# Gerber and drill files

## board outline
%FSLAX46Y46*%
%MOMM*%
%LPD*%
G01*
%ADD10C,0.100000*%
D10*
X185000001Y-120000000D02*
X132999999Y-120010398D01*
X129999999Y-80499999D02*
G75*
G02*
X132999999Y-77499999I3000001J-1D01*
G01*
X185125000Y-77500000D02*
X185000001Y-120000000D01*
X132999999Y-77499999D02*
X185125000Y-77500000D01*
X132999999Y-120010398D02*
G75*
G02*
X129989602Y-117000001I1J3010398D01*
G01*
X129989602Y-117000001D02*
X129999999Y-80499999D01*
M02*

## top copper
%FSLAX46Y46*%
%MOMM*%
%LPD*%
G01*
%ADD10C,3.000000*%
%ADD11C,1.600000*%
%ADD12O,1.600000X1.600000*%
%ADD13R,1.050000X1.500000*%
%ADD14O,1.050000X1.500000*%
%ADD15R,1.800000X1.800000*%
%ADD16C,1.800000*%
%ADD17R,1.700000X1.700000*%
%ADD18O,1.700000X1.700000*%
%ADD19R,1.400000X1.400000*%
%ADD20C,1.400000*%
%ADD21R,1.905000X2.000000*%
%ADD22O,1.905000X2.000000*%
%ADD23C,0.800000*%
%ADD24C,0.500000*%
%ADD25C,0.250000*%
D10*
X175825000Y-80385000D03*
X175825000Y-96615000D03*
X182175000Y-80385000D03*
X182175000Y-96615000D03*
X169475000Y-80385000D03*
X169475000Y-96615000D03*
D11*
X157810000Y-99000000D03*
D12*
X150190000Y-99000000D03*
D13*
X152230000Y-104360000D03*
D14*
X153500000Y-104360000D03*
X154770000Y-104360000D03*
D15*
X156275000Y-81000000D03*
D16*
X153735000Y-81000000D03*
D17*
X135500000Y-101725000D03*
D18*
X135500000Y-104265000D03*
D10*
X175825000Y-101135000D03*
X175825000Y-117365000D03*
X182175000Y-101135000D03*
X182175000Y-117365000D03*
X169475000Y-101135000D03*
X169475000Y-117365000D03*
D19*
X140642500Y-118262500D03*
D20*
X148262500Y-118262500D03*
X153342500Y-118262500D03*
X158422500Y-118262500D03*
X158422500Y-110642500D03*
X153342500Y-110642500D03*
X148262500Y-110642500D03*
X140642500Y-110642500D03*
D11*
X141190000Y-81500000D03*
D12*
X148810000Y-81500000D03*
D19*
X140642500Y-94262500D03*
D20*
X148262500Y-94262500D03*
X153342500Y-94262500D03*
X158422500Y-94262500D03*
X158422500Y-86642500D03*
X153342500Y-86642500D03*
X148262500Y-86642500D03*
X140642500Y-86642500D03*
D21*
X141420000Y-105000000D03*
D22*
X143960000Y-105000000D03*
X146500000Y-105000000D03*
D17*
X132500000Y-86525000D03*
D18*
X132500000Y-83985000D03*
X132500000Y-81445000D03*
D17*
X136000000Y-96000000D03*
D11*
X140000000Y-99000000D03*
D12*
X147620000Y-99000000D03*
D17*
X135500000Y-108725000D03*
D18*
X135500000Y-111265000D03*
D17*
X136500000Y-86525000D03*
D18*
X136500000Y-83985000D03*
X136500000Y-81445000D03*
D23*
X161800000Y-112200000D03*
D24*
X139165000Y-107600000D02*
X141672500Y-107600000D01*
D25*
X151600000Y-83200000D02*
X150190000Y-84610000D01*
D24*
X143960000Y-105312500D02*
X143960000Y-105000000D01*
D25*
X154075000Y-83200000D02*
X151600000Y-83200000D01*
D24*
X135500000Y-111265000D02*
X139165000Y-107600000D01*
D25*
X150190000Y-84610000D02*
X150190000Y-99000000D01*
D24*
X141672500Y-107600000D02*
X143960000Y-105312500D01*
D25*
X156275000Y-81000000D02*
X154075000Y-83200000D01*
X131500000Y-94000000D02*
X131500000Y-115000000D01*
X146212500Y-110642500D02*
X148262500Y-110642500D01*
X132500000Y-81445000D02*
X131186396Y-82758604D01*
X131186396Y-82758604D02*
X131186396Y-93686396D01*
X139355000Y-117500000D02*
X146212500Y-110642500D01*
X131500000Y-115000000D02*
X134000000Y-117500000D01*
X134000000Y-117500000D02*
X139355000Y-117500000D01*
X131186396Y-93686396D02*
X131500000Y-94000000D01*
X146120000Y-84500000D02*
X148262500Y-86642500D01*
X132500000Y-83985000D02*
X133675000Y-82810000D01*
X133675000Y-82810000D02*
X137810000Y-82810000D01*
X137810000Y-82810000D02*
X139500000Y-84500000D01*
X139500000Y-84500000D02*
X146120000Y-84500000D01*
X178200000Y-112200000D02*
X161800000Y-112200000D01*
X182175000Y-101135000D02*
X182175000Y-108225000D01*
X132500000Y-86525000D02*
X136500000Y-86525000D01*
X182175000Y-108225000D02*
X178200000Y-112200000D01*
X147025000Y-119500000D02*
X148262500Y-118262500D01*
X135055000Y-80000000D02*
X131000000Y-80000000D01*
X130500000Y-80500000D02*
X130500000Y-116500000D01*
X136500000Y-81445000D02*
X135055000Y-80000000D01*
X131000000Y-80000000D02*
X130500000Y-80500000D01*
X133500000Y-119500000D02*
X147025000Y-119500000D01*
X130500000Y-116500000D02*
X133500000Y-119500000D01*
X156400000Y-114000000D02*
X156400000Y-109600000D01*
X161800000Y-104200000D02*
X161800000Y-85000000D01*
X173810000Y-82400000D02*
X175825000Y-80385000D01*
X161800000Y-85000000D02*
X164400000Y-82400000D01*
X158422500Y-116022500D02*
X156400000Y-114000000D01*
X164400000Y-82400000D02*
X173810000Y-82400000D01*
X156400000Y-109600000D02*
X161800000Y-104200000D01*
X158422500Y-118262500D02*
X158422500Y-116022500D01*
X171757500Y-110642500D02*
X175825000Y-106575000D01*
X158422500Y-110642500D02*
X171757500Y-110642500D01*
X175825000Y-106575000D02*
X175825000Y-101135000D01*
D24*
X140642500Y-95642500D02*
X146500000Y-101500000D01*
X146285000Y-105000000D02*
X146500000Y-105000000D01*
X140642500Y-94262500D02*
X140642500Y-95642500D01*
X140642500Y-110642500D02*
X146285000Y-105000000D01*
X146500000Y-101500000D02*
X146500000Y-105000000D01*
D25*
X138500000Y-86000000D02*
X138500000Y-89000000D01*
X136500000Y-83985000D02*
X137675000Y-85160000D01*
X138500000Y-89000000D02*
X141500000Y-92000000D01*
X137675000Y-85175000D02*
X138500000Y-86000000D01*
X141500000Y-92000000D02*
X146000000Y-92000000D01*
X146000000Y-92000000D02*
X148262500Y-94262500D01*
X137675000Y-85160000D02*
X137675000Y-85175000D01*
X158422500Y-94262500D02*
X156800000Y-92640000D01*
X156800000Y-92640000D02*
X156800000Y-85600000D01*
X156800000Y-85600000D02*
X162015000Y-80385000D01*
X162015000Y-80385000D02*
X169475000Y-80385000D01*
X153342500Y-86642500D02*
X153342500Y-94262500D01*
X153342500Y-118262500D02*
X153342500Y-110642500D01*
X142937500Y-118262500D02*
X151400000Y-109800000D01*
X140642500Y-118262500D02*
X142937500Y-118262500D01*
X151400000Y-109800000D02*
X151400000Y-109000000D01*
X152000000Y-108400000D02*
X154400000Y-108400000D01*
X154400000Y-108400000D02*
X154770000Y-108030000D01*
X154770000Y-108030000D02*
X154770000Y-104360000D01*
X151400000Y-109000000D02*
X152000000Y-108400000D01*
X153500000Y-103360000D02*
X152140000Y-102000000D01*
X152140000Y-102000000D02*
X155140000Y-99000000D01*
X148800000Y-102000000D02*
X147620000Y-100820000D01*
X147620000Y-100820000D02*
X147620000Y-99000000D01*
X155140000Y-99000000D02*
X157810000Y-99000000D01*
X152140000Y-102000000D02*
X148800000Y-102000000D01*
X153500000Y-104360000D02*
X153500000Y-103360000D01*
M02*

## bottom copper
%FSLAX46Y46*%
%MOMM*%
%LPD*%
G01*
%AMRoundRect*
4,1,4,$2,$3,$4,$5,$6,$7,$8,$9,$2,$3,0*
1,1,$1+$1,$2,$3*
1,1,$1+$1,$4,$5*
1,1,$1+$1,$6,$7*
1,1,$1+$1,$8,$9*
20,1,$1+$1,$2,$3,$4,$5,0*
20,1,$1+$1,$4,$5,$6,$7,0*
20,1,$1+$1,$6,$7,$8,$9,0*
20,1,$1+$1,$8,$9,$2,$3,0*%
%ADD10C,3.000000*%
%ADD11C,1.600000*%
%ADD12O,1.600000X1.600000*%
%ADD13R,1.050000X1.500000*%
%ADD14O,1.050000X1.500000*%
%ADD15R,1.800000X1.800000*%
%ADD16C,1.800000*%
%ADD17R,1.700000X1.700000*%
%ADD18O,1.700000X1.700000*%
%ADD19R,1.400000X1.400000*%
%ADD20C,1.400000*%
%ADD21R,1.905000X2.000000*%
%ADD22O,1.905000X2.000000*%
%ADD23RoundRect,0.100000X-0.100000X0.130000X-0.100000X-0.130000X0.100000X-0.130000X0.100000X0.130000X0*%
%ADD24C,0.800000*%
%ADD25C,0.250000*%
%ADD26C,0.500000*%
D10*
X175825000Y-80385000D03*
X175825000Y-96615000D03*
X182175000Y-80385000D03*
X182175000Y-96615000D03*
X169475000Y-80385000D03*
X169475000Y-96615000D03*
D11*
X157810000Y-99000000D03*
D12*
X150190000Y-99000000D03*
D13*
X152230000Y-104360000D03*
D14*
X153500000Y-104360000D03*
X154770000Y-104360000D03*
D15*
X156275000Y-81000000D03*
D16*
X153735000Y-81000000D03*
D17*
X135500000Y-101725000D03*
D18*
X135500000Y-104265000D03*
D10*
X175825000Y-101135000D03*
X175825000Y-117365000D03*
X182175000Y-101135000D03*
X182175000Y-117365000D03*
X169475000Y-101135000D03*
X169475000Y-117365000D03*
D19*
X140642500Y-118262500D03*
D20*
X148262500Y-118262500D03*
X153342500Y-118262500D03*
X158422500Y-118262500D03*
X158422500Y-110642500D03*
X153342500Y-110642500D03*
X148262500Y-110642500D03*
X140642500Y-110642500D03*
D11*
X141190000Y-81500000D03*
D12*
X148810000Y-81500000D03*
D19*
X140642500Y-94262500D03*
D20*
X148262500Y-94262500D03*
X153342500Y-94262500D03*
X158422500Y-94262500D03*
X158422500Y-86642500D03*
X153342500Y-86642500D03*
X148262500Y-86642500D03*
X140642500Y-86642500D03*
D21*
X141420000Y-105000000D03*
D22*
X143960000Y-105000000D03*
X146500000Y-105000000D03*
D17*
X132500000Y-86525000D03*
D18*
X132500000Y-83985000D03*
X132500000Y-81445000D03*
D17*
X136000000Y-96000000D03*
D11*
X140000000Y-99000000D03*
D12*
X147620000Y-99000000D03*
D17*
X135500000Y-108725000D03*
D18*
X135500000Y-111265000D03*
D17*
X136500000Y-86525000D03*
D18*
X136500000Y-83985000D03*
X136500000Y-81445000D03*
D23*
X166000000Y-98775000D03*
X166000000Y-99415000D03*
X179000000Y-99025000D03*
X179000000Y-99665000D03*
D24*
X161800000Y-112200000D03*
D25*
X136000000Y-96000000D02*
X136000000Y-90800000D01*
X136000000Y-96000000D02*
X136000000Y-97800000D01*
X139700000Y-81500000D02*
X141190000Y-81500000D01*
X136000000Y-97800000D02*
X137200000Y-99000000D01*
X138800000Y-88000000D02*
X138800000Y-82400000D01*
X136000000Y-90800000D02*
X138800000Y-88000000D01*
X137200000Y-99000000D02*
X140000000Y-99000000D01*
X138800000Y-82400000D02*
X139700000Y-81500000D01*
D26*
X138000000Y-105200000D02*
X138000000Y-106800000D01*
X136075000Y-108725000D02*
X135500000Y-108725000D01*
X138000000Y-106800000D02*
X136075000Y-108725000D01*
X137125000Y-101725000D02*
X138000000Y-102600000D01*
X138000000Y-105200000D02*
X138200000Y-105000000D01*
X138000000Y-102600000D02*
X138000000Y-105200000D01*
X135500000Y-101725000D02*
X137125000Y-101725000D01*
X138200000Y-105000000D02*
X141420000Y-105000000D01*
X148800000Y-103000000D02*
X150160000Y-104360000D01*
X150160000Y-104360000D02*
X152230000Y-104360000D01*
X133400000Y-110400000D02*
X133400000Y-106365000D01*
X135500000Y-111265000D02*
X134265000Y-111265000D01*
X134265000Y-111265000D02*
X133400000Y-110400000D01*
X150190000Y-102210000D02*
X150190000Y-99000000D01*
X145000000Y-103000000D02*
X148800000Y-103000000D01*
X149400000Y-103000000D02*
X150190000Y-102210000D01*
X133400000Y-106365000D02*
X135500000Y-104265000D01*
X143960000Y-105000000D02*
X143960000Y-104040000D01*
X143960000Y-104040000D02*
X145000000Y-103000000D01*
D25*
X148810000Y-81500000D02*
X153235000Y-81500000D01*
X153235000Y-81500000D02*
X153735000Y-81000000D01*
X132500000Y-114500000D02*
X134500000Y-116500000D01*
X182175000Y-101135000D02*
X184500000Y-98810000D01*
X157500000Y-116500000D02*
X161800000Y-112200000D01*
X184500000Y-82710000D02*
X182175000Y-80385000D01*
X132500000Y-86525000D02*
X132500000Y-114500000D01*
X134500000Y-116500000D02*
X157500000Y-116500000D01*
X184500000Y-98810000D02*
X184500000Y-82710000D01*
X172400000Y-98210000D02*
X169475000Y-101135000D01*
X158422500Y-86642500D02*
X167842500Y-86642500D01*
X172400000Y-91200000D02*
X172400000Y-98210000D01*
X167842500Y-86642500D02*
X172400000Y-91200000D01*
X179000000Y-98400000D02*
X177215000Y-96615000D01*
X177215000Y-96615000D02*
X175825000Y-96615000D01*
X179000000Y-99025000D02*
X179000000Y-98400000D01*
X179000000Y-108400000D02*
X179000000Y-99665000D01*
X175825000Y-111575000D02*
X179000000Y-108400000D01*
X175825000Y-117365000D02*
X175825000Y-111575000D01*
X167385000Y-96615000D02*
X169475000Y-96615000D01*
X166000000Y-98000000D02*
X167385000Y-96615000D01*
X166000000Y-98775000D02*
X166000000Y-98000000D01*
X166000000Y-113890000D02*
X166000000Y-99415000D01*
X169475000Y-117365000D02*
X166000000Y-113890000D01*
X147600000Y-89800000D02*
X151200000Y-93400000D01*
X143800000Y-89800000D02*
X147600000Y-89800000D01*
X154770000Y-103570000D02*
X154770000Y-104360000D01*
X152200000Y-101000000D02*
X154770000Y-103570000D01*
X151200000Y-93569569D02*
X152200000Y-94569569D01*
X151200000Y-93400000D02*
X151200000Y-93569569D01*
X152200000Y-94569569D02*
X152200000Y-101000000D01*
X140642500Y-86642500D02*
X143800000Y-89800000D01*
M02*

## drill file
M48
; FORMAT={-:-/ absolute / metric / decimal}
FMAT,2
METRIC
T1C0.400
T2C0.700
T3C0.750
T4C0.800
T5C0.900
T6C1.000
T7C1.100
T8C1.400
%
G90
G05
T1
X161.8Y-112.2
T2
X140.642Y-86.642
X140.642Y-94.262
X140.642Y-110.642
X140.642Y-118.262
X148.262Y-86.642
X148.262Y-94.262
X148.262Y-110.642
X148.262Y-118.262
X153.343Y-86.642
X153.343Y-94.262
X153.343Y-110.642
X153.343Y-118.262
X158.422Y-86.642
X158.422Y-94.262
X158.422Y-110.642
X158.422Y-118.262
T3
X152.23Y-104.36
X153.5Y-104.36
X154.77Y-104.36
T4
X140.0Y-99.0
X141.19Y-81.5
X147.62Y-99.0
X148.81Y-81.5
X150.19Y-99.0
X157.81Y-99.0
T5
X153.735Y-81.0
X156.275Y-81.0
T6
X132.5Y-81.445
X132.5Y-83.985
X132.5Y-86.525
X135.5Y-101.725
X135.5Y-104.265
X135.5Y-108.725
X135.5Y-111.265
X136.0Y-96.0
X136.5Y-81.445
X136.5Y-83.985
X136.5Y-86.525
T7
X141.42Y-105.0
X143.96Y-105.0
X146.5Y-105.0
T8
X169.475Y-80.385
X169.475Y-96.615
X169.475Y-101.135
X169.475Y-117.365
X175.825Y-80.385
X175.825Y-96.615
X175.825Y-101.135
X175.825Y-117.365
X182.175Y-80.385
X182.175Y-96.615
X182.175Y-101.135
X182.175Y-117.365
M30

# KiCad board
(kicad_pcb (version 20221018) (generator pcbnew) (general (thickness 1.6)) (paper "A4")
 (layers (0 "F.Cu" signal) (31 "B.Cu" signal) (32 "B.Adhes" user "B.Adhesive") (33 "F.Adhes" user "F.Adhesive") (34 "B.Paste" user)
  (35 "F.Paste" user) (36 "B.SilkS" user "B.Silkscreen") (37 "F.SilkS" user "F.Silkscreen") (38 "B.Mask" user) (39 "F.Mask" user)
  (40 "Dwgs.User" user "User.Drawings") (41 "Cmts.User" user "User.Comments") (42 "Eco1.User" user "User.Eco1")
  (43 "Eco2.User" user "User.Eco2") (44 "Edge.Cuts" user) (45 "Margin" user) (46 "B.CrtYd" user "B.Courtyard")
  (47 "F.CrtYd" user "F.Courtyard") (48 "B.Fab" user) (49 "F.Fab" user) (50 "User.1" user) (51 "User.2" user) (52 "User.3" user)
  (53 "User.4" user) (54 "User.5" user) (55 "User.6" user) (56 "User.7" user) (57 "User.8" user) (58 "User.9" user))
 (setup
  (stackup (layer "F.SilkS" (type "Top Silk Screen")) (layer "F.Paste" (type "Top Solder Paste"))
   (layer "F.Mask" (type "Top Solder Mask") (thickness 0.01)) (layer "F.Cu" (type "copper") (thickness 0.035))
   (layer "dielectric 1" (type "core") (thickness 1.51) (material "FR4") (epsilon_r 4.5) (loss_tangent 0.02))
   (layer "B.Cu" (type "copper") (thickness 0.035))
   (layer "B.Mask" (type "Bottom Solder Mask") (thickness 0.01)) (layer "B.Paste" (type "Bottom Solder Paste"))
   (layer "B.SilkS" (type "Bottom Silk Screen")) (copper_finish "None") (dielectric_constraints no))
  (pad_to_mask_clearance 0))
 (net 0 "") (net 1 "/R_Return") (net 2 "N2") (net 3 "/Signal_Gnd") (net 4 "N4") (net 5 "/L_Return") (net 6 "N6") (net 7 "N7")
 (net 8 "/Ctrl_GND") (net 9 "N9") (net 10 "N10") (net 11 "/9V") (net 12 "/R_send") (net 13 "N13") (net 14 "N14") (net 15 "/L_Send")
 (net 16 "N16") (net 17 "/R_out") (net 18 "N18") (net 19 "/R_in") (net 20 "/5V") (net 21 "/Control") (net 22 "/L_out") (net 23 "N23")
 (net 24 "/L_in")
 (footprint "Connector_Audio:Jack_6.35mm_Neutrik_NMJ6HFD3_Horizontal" (layer "F.Cu") (at 169.475 80.385)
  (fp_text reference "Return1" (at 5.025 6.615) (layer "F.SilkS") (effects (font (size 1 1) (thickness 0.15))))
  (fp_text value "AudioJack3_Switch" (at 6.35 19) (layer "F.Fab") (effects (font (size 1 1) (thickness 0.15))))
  (pad "R" thru_hole circle (at 6.35 0) (size 3 3) (drill 1.4) (layers "*.Cu" "*.Mask") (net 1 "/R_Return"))
  (pad "RN" thru_hole circle (at 6.35 16.23) (size 3 3) (drill 1.4) (layers "*.Cu" "*.Mask") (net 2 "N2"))
  (pad "S" thru_hole circle (at 12.7 0) (size 3 3) (drill 1.4) (layers "*.Cu" "*.Mask") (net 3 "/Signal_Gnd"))
  (pad "SN" thru_hole circle (at 12.7 16.23) (size 3 3) (drill 1.4) (layers "*.Cu" "*.Mask") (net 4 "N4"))
  (pad "T" thru_hole circle (at 0 0) (size 3 3) (drill 1.4) (layers "*.Cu" "*.Mask") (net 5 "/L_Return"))
  (pad "TN" thru_hole circle (at 0 16.23) (size 3 3) (drill 1.4) (layers "*.Cu" "*.Mask") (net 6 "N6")))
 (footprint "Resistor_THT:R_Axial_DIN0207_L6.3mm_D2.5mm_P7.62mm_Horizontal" (layer "F.Cu") (at 157.81 99 180)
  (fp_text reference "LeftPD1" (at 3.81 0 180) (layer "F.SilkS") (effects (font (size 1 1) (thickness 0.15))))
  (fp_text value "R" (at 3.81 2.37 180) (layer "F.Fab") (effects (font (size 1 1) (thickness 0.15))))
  (pad "1" thru_hole circle (at 0 0 180) (size 1.6 1.6) (drill 0.8) (layers "*.Cu" "*.Mask") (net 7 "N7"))
  (pad "2" thru_hole oval (at 7.62 0 180) (size 1.6 1.6) (drill 0.8) (layers "*.Cu" "*.Mask") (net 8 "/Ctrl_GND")))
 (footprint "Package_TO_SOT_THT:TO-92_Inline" (layer "F.Cu") (at 152.23 104.36)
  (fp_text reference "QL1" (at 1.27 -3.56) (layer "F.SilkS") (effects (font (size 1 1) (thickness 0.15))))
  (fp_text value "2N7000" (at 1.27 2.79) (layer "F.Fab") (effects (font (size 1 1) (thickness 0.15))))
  (pad "1" thru_hole rect (at 0 0) (size 1.05 1.5) (drill 0.75) (layers "*.Cu" "*.Mask") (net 8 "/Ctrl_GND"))
  (pad "2" thru_hole oval (at 1.27 0) (size 1.05 1.5) (drill 0.75) (layers "*.Cu" "*.Mask") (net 7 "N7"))
  (pad "3" thru_hole oval (at 2.54 0) (size 1.05 1.5) (drill 0.75) (layers "*.Cu" "*.Mask") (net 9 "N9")))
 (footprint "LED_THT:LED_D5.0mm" (layer "F.Cu") (at 156.275 81 180)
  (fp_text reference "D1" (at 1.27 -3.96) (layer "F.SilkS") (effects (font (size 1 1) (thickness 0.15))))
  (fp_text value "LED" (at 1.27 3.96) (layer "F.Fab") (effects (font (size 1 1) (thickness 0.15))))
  (pad "1" thru_hole rect (at 0 0 180) (size 1.8 1.8) (drill 0.9) (layers "*.Cu" "*.Mask") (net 8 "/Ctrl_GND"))
  (pad "2" thru_hole circle (at 2.54 0 180) (size 1.8 1.8) (drill 0.9) (layers "*.Cu" "*.Mask") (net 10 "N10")))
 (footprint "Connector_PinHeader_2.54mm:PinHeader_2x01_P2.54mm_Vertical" (layer "F.Cu") (at 135.5 101.725 -90)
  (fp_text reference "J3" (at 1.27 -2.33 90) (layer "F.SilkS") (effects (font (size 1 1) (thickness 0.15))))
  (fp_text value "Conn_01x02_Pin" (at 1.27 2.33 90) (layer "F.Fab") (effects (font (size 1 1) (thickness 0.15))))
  (pad "1" thru_hole rect (at 0 0 270) (size 1.7 1.7) (drill 1) (layers "*.Cu" "*.Mask") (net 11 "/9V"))
  (pad "2" thru_hole oval (at 2.54 0 270) (size 1.7 1.7) (drill 1) (layers "*.Cu" "*.Mask") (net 8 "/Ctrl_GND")))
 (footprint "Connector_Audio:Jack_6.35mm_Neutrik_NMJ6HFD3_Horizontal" (layer "F.Cu") (at 169.475 101.135)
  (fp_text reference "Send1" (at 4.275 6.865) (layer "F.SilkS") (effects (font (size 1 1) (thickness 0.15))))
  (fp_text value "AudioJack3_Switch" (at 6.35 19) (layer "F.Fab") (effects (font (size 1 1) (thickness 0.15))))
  (pad "R" thru_hole circle (at 6.35 0) (size 3 3) (drill 1.4) (layers "*.Cu" "*.Mask") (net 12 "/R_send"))
  (pad "RN" thru_hole circle (at 6.35 16.23) (size 3 3) (drill 1.4) (layers "*.Cu" "*.Mask") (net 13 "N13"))
  (pad "S" thru_hole circle (at 12.7 0) (size 3 3) (drill 1.4) (layers "*.Cu" "*.Mask") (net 3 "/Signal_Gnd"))
  (pad "SN" thru_hole circle (at 12.7 16.23) (size 3 3) (drill 1.4) (layers "*.Cu" "*.Mask") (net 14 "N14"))
  (pad "T" thru_hole circle (at 0 0) (size 3 3) (drill 1.4) (layers "*.Cu" "*.Mask") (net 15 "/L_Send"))
  (pad "TN" thru_hole circle (at 0 16.23) (size 3 3) (drill 1.4) (layers "*.Cu" "*.Mask") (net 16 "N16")))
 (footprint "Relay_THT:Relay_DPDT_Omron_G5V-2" (layer "F.Cu") (at 140.6425 118.2625 90)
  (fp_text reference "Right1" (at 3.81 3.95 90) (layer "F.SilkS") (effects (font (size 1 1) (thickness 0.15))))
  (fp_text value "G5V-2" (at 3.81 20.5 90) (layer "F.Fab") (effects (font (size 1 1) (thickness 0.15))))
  (pad "1" thru_hole rect (at 0 0 90) (size 1.4 1.4) (drill 0.7) (layers "*.Cu" "*.Mask") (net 9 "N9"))
  (pad "4" thru_hole circle (at 0 7.62 90) (size 1.4 1.4) (drill 0.7) (layers "*.Cu" "*.Mask") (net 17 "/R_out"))
  (pad "6" thru_hole circle (at 0 12.7 90) (size 1.4 1.4) (drill 0.7) (layers "*.Cu" "*.Mask") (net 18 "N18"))
  (pad "8" thru_hole circle (at 0 17.78 90) (size 1.4 1.4) (drill 0.7) (layers "*.Cu" "*.Mask") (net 1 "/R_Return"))
  (pad "9" thru_hole circle (at 7.62 17.78 90) (size 1.4 1.4) (drill 0.7) (layers "*.Cu" "*.Mask") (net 12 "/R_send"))
  (pad "11" thru_hole circle (at 7.62 12.7 90) (size 1.4 1.4) (drill 0.7) (layers "*.Cu" "*.Mask") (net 18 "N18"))
  (pad "13" thru_hole circle (at 7.62 7.62 90) (size 1.4 1.4) (drill 0.7) (layers "*.Cu" "*.Mask") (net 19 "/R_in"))
  (pad "16" thru_hole circle (at 7.62 0 90) (size 1.4 1.4) (drill 0.7) (layers "*.Cu" "*.Mask") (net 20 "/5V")))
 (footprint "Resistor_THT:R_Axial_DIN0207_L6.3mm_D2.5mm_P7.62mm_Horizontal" (layer "F.Cu") (at 141.19 81.5)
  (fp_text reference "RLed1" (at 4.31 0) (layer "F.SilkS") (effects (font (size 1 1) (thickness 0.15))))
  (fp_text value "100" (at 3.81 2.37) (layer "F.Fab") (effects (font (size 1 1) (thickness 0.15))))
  (pad "1" thru_hole circle (at 0 0) (size 1.6 1.6) (drill 0.8) (layers "*.Cu" "*.Mask") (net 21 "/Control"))
  (pad "2" thru_hole oval (at 7.62 0) (size 1.6 1.6) (drill 0.8) (layers "*.Cu" "*.Mask") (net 10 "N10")))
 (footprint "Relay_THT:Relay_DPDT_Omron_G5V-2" (layer "F.Cu") (at 140.6425 94.2625 90)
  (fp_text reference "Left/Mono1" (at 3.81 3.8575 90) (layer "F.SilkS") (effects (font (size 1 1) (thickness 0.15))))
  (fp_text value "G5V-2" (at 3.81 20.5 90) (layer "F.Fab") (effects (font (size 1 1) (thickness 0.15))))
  (pad "1" thru_hole rect (at 0 0 90) (size 1.4 1.4) (drill 0.7) (layers "*.Cu" "*.Mask") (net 20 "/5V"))
  (pad "4" thru_hole circle (at 0 7.62 90) (size 1.4 1.4) (drill 0.7) (layers "*.Cu" "*.Mask") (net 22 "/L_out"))
  (pad "6" thru_hole circle (at 0 12.7 90) (size 1.4 1.4) (drill 0.7) (layers "*.Cu" "*.Mask") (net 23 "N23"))
  (pad "8" thru_hole circle (at 0 17.78 90) (size 1.4 1.4) (drill 0.7) (layers "*.Cu" "*.Mask") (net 5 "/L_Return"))
  (pad "9" thru_hole circle (at 7.62 17.78 90) (size 1.4 1.4) (drill 0.7) (layers "*.Cu" "*.Mask") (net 15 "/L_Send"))
  (pad "11" thru_hole circle (at 7.62 12.7 90) (size 1.4 1.4) (drill 0.7) (layers "*.Cu" "*.Mask") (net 23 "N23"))
  (pad "13" thru_hole circle (at 7.62 7.62 90) (size 1.4 1.4) (drill 0.7) (layers "*.Cu" "*.Mask") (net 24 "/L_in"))
  (pad "16" thru_hole circle (at 7.62 0 90) (size 1.4 1.4) (drill 0.7) (layers "*.Cu" "*.Mask") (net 9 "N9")))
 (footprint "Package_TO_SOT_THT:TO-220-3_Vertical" (layer "F.Cu") (at 141.42 105)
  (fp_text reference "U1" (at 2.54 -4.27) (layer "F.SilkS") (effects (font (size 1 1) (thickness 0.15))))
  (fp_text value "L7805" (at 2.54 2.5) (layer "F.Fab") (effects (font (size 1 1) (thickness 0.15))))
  (pad "1" thru_hole rect (at 0 0) (size 1.905 2) (drill 1.1) (layers "*.Cu" "*.Mask") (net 11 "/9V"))
  (pad "2" thru_hole oval (at 2.54 0) (size 1.905 2) (drill 1.1) (layers "*.Cu" "*.Mask") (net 8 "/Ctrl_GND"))
  (pad "3" thru_hole oval (at 5.08 0) (size 1.905 2) (drill 1.1) (layers "*.Cu" "*.Mask") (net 20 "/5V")))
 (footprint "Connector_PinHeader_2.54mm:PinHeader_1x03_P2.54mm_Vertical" (layer "F.Cu") (at 132.5 86.525 180)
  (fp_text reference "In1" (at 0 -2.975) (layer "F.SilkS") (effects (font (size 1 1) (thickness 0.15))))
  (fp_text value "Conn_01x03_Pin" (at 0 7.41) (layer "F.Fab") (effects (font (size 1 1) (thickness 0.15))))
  (pad "1" thru_hole rect (at 0 0 180) (size 1.7 1.7) (drill 1) (layers "*.Cu" "*.Mask") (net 3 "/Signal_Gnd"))
  (pad "2" thru_hole oval (at 0 2.54 180) (size 1.7 1.7) (drill 1) (layers "*.Cu" "*.Mask") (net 24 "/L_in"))
  (pad "3" thru_hole oval (at 0 5.08 180) (size 1.7 1.7) (drill 1) (layers "*.Cu" "*.Mask") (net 19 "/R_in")))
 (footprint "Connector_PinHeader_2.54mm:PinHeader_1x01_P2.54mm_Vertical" (layer "F.Cu") (at 136 96)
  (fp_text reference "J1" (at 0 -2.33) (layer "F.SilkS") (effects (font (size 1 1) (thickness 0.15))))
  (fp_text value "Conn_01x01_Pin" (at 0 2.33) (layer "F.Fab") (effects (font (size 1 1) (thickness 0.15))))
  (pad "1" thru_hole rect (at 0 0) (size 1.7 1.7) (drill 1) (layers "*.Cu" "*.Mask") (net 21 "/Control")))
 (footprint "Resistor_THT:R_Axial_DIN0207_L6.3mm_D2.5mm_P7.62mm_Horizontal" (layer "F.Cu") (at 140 99)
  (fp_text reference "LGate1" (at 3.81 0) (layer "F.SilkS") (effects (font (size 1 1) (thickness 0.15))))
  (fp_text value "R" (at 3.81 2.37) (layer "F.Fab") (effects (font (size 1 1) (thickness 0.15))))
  (pad "1" thru_hole circle (at 0 0) (size 1.6 1.6) (drill 0.8) (layers "*.Cu" "*.Mask") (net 21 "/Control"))
  (pad "2" thru_hole oval (at 7.62 0) (size 1.6 1.6) (drill 0.8) (layers "*.Cu" "*.Mask") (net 7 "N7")))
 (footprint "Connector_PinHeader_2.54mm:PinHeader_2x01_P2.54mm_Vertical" (layer "F.Cu") (at 135.5 108.725 -90)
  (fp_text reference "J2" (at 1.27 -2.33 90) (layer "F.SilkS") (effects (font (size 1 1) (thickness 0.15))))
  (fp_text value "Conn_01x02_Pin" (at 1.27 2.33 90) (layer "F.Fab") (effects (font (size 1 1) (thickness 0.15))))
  (pad "1" thru_hole rect (at 0 0 270) (size 1.7 1.7) (drill 1) (layers "*.Cu" "*.Mask") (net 11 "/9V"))
  (pad "2" thru_hole oval (at 2.54 0 270) (size 1.7 1.7) (drill 1) (layers "*.Cu" "*.Mask") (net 8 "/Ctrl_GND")))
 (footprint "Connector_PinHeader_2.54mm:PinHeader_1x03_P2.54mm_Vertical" (layer "F.Cu") (at 136.5 86.525 180)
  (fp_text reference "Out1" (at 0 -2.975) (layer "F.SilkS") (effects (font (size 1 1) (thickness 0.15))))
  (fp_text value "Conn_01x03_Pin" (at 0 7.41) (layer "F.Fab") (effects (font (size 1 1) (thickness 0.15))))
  (pad "1" thru_hole rect (at 0 0 180) (size 1.7 1.7) (drill 1) (layers "*.Cu" "*.Mask") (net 3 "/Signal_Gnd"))
  (pad "2" thru_hole oval (at 0 2.54 180) (size 1.7 1.7) (drill 1) (layers "*.Cu" "*.Mask") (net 22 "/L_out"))
  (pad "3" thru_hole oval (at 0 5.08 180) (size 1.7 1.7) (drill 1) (layers "*.Cu" "*.Mask") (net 17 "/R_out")))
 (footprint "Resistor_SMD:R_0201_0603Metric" (layer "B.Cu") (at 166 99.095 -90)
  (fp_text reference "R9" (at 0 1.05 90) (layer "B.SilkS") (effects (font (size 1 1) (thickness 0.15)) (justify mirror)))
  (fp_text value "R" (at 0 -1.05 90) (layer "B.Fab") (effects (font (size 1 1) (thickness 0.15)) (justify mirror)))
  (pad "" smd roundrect (at -0.345 0 270) (size 0.318 0.36) (layers "B.Paste") (roundrect_rratio 0.25))
  (pad "" smd roundrect (at 0.345 0 270) (size 0.318 0.36) (layers "B.Paste") (roundrect_rratio 0.25))
  (pad "1" smd roundrect (at -0.32 0 270) (size 0.46 0.4) (layers "B.Cu" "B.Mask") (roundrect_rratio 0.25) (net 6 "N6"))
  (pad "2" smd roundrect (at 0.32 0 270) (size 0.46 0.4) (layers "B.Cu" "B.Mask") (roundrect_rratio 0.25) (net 16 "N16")))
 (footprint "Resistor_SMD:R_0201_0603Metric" (layer "B.Cu") (at 179 99.345 -90)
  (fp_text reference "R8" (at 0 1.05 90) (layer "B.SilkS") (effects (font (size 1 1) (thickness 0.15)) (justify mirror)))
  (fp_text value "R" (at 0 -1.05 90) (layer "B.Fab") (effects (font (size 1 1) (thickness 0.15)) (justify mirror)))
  (pad "" smd roundrect (at -0.345 0 270) (size 0.318 0.36) (layers "B.Paste") (roundrect_rratio 0.25))
  (pad "" smd roundrect (at 0.345 0 270) (size 0.318 0.36) (layers "B.Paste") (roundrect_rratio 0.25))
  (pad "1" smd roundrect (at -0.32 0 270) (size 0.46 0.4) (layers "B.Cu" "B.Mask") (roundrect_rratio 0.25) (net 2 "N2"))
  (pad "2" smd roundrect (at 0.32 0 270) (size 0.46 0.4) (layers "B.Cu" "B.Mask") (roundrect_rratio 0.25) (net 13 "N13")))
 (gr_line (start 185.000001 120) (end 132.999999 120.010398) (stroke (width 0.1) (type default)) (layer "Edge.Cuts"))
 (gr_arc (start 129.999999 80.499999) (mid 130.878679 78.378679) (end 132.999999 77.499999) (stroke (width 0.1) (type default))
  (layer "Edge.Cuts"))
 (gr_line (start 185.125 77.5) (end 185.000001 120) (stroke (width 0.1) (type default)) (layer "Edge.Cuts"))
 (gr_line (start 132.999999 77.499999) (end 185.125 77.5) (stroke (width 0.1) (type default)) (layer "Edge.Cuts"))
 (gr_arc (start 132.999999 120.010398) (mid 130.871327 119.128673) (end 129.989602 117.000001) (stroke (width 0.1) (type default))
  (layer "Edge.Cuts"))
 (gr_line (start 129.989602 117.000001) (end 129.999999 80.499999) (stroke (width 0.1) (type default)) (layer "Edge.Cuts"))
 (segment (start 136 96) (end 136 90.8) (width 0.25) (layer "B.Cu") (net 21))
 (segment (start 136 96) (end 136 97.8) (width 0.25) (layer "B.Cu") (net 21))
 (segment (start 139.7 81.5) (end 141.19 81.5) (width 0.25) (layer "B.Cu") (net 21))
 (segment (start 136 97.8) (end 137.2 99) (width 0.25) (layer "B.Cu") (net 21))
 (segment (start 138.8 88) (end 138.8 82.4) (width 0.25) (layer "B.Cu") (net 21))
 (segment (start 136 90.8) (end 138.8 88) (width 0.25) (layer "B.Cu") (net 21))
 (segment (start 137.2 99) (end 140 99) (width 0.25) (layer "B.Cu") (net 21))
 (segment (start 138.8 82.4) (end 139.7 81.5) (width 0.25) (layer "B.Cu") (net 21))
 (segment (start 138 105.2) (end 138 106.8) (width 0.5) (layer "B.Cu") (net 11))
 (segment (start 136.075 108.725) (end 135.5 108.725) (width 0.5) (layer "B.Cu") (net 11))
 (segment (start 138 106.8) (end 136.075 108.725) (width 0.5) (layer "B.Cu") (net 11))
 (segment (start 137.125 101.725) (end 138 102.6) (width 0.5) (layer "B.Cu") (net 11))
 (segment (start 138 105.2) (end 138.2 105) (width 0.5) (layer "B.Cu") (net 11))
 (segment (start 138 102.6) (end 138 105.2) (width 0.5) (layer "B.Cu") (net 11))
 (segment (start 135.5 101.725) (end 137.125 101.725) (width 0.5) (layer "B.Cu") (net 11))
 (segment (start 138.2 105) (end 141.42 105) (width 0.5) (layer "B.Cu") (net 11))
 (segment (start 139.165 107.6) (end 141.6725 107.6) (width 0.5) (layer "F.Cu") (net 8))
 (segment (start 151.6 83.2) (end 150.19 84.61) (width 0.25) (layer "F.Cu") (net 8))
 (segment (start 143.96 105.3125) (end 143.96 105) (width 0.5) (layer "F.Cu") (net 8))
 (segment (start 154.075 83.2) (end 151.6 83.2) (width 0.25) (layer "F.Cu") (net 8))
 (segment (start 135.5 111.265) (end 139.165 107.6) (width 0.5) (layer "F.Cu") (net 8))
 (segment (start 150.19 84.61) (end 150.19 99) (width 0.25) (layer "F.Cu") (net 8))
 (segment (start 141.6725 107.6) (end 143.96 105.3125) (width 0.5) (layer "F.Cu") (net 8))
 (segment (start 156.275 81) (end 154.075 83.2) (width 0.25) (layer "F.Cu") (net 8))
 (segment (start 148.8 103) (end 150.16 104.36) (width 0.5) (layer "B.Cu") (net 8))
 (segment (start 150.16 104.36) (end 152.23 104.36) (width 0.5) (layer "B.Cu") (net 8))
 (segment (start 133.4 110.4) (end 133.4 106.365) (width 0.5) (layer "B.Cu") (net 8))
 (segment (start 135.5 111.265) (end 134.265 111.265) (width 0.5) (layer "B.Cu") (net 8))
 (segment (start 134.265 111.265) (end 133.4 110.4) (width 0.5) (layer "B.Cu") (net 8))
 (segment (start 150.19 102.21) (end 150.19 99) (width 0.5) (layer "B.Cu") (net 8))
 (segment (start 145 103) (end 148.8 103) (width 0.5) (layer "B.Cu") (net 8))
 (segment (start 149.4 103) (end 150.19 102.21) (width 0.5) (layer "B.Cu") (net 8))
 (segment (start 133.4 106.365) (end 135.5 104.265) (width 0.5) (layer "B.Cu") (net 8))
 (segment (start 143.96 105) (end 143.96 104.04) (width 0.5) (layer "B.Cu") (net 8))
 (segment (start 143.96 104.04) (end 145 103) (width 0.5) (layer "B.Cu") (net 8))
 (segment (start 148.81 81.5) (end 153.235 81.5) (width 0.25) (layer "B.Cu") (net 10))
 (segment (start 153.235 81.5) (end 153.735 81) (width 0.25) (layer "B.Cu") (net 10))
 (segment (start 131.5 94) (end 131.5 115) (width 0.25) (layer "F.Cu") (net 19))
 (segment (start 146.2125 110.6425) (end 148.2625 110.6425) (width 0.25) (layer "F.Cu") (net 19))
 (segment (start 132.5 81.445) (end 131.186396 82.758604) (width 0.25) (layer "F.Cu") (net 19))
 (segment (start 131.186396 82.758604) (end 131.186396 93.686396) (width 0.25) (layer "F.Cu") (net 19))
 (segment (start 139.355 117.5) (end 146.2125 110.6425) (width 0.25) (layer "F.Cu") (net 19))
 (segment (start 131.5 115) (end 134 117.5) (width 0.25) (layer "F.Cu") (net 19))
 (segment (start 134 117.5) (end 139.355 117.5) (width 0.25) (layer "F.Cu") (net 19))
 (segment (start 131.186396 93.686396) (end 131.5 94) (width 0.25) (layer "F.Cu") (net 19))
 (segment (start 146.12 84.5) (end 148.2625 86.6425) (width 0.25) (layer "F.Cu") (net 24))
 (segment (start 132.5 83.985) (end 133.675 82.81) (width 0.25) (layer "F.Cu") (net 24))
 (segment (start 133.675 82.81) (end 137.81 82.81) (width 0.25) (layer "F.Cu") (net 24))
 (segment (start 137.81 82.81) (end 139.5 84.5) (width 0.25) (layer "F.Cu") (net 24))
 (segment (start 139.5 84.5) (end 146.12 84.5) (width 0.25) (layer "F.Cu") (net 24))
 (segment (start 178.2 112.2) (end 161.8 112.2) (width 0.25) (layer "F.Cu") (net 3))
 (segment (start 182.175 101.135) (end 182.175 108.225) (width 0.25) (layer "F.Cu") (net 3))
 (segment (start 132.5 86.525) (end 136.5 86.525) (width 0.25) (layer "F.Cu") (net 3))
 (segment (start 182.175 108.225) (end 178.2 112.2) (width 0.25) (layer "F.Cu") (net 3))
 (via (at 161.8 112.2) (size 0.8) (drill 0.4) (layers "F.Cu" "B.Cu") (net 3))
 (segment (start 132.5 114.5) (end 134.5 116.5) (width 0.25) (layer "B.Cu") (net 3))
 (segment (start 182.175 101.135) (end 184.5 98.81) (width 0.25) (layer "B.Cu") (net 3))
 (segment (start 157.5 116.5) (end 161.8 112.2) (width 0.25) (layer "B.Cu") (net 3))
 (segment (start 184.5 82.71) (end 182.175 80.385) (width 0.25) (layer "B.Cu") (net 3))
 (segment (start 132.5 86.525) (end 132.5 114.5) (width 0.25) (layer "B.Cu") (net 3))
 (segment (start 134.5 116.5) (end 157.5 116.5) (width 0.25) (layer "B.Cu") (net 3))
 (segment (start 184.5 98.81) (end 184.5 82.71) (width 0.25) (layer "B.Cu") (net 3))
 (segment (start 147.025 119.5) (end 148.2625 118.2625) (width 0.25) (layer "F.Cu") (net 17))
 (segment (start 135.055 80) (end 131 80) (width 0.25) (layer "F.Cu") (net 17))
 (segment (start 130.5 80.5) (end 130.5 116.5) (width 0.25) (layer "F.Cu") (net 17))
 (segment (start 136.5 81.445) (end 135.055 80) (width 0.25) (layer "F.Cu") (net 17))
 (segment (start 131 80) (end 130.5 80.5) (width 0.25) (layer "F.Cu") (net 17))
 (segment (start 133.5 119.5) (end 147.025 119.5) (width 0.25) (layer "F.Cu") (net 17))
 (segment (start 130.5 116.5) (end 133.5 119.5) (width 0.25) (layer "F.Cu") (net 17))
 (segment (start 156.4 114) (end 156.4 109.6) (width 0.25) (layer "F.Cu") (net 1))
 (segment (start 161.8 104.2) (end 161.8 85) (width 0.25) (layer "F.Cu") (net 1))
 (segment (start 173.81 82.4) (end 175.825 80.385) (width 0.25) (layer "F.Cu") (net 1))
 (segment (start 161.8 85) (end 164.4 82.4) (width 0.25) (layer "F.Cu") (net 1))
 (segment (start 158.4225 116.0225) (end 156.4 114) (width 0.25) (layer "F.Cu") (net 1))
 (segment (start 164.4 82.4) (end 173.81 82.4) (width 0.25) (layer "F.Cu") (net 1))
 (segment (start 156.4 109.6) (end 161.8 104.2) (width 0.25) (layer "F.Cu") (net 1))
 (segment (start 158.4225 118.2625) (end 158.4225 116.0225) (width 0.25) (layer "F.Cu") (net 1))
 (segment (start 171.7575 110.6425) (end 175.825 106.575) (width 0.25) (layer "F.Cu") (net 12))
 (segment (start 158.4225 110.6425) (end 171.7575 110.6425) (width 0.25) (layer "F.Cu") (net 12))
 (segment (start 175.825 106.575) (end 175.825 101.135) (width 0.25) (layer "F.Cu") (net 12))
 (segment (start 140.6425 95.6425) (end 146.5 101.5) (width 0.5) (layer "F.Cu") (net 20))
 (segment (start 146.285 105) (end 146.5 105) (width 0.5) (layer "F.Cu") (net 20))
 (segment (start 140.6425 94.2625) (end 140.6425 95.6425) (width 0.5) (layer "F.Cu") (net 20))
 (segment (start 140.6425 110.6425) (end 146.285 105) (width 0.5) (layer "F.Cu") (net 20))
 (segment (start 146.5 101.5) (end 146.5 105) (width 0.5) (layer "F.Cu") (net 20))
 (segment (start 138.5 86) (end 138.5 89) (width 0.25) (layer "F.Cu") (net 22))
 (segment (start 136.5 83.985) (end 137.675 85.16) (width 0.25) (layer "F.Cu") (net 22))
 (segment (start 138.5 89) (end 141.5 92) (width 0.25) (layer "F.Cu") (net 22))
 (segment (start 137.675 85.175) (end 138.5 86) (width 0.25) (layer "F.Cu") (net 22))
 (segment (start 141.5 92) (end 146 92) (width 0.25) (layer "F.Cu") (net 22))
 (segment (start 146 92) (end 148.2625 94.2625) (width 0.25) (layer "F.Cu") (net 22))
 (segment (start 137.675 85.16) (end 137.675 85.175) (width 0.25) (layer "F.Cu") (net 22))
 (segment (start 158.4225 94.2625) (end 156.8 92.64) (width 0.25) (layer "F.Cu") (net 5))
 (segment (start 156.8 92.64) (end 156.8 85.6) (width 0.25) (layer "F.Cu") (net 5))
 (segment (start 156.8 85.6) (end 162.015 80.385) (width 0.25) (layer "F.Cu") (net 5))
 (segment (start 162.015 80.385) (end 169.475 80.385) (width 0.25) (layer "F.Cu") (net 5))
 (segment (start 172.4 98.21) (end 169.475 101.135) (width 0.25) (layer "B.Cu") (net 15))
 (segment (start 158.4225 86.6425) (end 167.8425 86.6425) (width 0.25) (layer "B.Cu") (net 15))
 (segment (start 172.4 91.2) (end 172.4 98.21) (width 0.25) (layer "B.Cu") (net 15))
 (segment (start 167.8425 86.6425) (end 172.4 91.2) (width 0.25) (layer "B.Cu") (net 15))
 (segment (start 179 98.4) (end 177.215 96.615) (width 0.25) (layer "B.Cu") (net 2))
 (segment (start 177.215 96.615) (end 175.825 96.615) (width 0.25) (layer "B.Cu") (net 2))
 (segment (start 179 99.025) (end 179 98.4) (width 0.25) (layer "B.Cu") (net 2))
 (segment (start 179 108.4) (end 179 99.665) (width 0.25) (layer "B.Cu") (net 13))
 (segment (start 175.825 111.575) (end 179 108.4) (width 0.25) (layer "B.Cu") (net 13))
 (segment (start 175.825 117.365) (end 175.825 111.575) (width 0.25) (layer "B.Cu") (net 13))
 (segment (start 167.385 96.615) (end 169.475 96.615) (width 0.25) (layer "B.Cu") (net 6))
 (segment (start 166 98) (end 167.385 96.615) (width 0.25) (layer "B.Cu") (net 6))
 (segment (start 166 98.775) (end 166 98) (width 0.25) (layer "B.Cu") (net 6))
 (segment (start 166 113.89) (end 166 99.415) (width 0.25) (layer "B.Cu") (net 16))
 (segment (start 169.475 117.365) (end 166 113.89) (width 0.25) (layer "B.Cu") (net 16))
 (segment (start 153.3425 86.6425) (end 153.3425 94.2625) (width 0.25) (layer "F.Cu") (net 23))
 (segment (start 153.3425 118.2625) (end 153.3425 110.6425) (width 0.25) (layer "F.Cu") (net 18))
 (segment (start 142.9375 118.2625) (end 151.4 109.8) (width 0.25) (layer "F.Cu") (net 9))
 (segment (start 140.6425 118.2625) (end 142.9375 118.2625) (width 0.25) (layer "F.Cu") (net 9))
 (segment (start 151.4 109.8) (end 151.4 109) (width 0.25) (layer "F.Cu") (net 9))
 (segment (start 152 108.4) (end 154.4 108.4) (width 0.25) (layer "F.Cu") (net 9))
 (segment (start 154.4 108.4) (end 154.77 108.03) (width 0.25) (layer "F.Cu") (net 9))
 (segment (start 154.77 108.03) (end 154.77 104.36) (width 0.25) (layer "F.Cu") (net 9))
 (segment (start 151.4 109) (end 152 108.4) (width 0.25) (layer "F.Cu") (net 9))
 (segment (start 147.6 89.8) (end 151.2 93.4) (width 0.25) (layer "B.Cu") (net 9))
 (segment (start 143.8 89.8) (end 147.6 89.8) (width 0.25) (layer "B.Cu") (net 9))
 (segment (start 154.77 103.57) (end 154.77 104.36) (width 0.25) (layer "B.Cu") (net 9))
 (segment (start 152.2 101) (end 154.77 103.57) (width 0.25) (layer "B.Cu") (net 9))
 (segment (start 151.2 93.569569) (end 152.2 94.569569) (width 0.25) (layer "B.Cu") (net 9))
 (segment (start 151.2 93.4) (end 151.2 93.569569) (width 0.25) (layer "B.Cu") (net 9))
 (segment (start 152.2 94.569569) (end 152.2 101) (width 0.25) (layer "B.Cu") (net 9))
 (segment (start 140.6425 86.6425) (end 143.8 89.8) (width 0.25) (layer "B.Cu") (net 9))
 (segment (start 153.5 103.36) (end 152.14 102) (width 0.25) (layer "F.Cu") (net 7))
 (segment (start 152.14 102) (end 155.14 99) (width 0.25) (layer "F.Cu") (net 7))
 (segment (start 148.8 102) (end 147.62 100.82) (width 0.25) (layer "F.Cu") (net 7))
 (segment (start 147.62 100.82) (end 147.62 99) (width 0.25) (layer "F.Cu") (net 7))
 (segment (start 155.14 99) (end 157.81 99) (width 0.25) (layer "F.Cu") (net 7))
 (segment (start 152.14 102) (end 148.8 102) (width 0.25) (layer "F.Cu") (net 7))
 (segment (start 153.5 104.36) (end 153.5 103.36) (width 0.25) (layer "F.Cu") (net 7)))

